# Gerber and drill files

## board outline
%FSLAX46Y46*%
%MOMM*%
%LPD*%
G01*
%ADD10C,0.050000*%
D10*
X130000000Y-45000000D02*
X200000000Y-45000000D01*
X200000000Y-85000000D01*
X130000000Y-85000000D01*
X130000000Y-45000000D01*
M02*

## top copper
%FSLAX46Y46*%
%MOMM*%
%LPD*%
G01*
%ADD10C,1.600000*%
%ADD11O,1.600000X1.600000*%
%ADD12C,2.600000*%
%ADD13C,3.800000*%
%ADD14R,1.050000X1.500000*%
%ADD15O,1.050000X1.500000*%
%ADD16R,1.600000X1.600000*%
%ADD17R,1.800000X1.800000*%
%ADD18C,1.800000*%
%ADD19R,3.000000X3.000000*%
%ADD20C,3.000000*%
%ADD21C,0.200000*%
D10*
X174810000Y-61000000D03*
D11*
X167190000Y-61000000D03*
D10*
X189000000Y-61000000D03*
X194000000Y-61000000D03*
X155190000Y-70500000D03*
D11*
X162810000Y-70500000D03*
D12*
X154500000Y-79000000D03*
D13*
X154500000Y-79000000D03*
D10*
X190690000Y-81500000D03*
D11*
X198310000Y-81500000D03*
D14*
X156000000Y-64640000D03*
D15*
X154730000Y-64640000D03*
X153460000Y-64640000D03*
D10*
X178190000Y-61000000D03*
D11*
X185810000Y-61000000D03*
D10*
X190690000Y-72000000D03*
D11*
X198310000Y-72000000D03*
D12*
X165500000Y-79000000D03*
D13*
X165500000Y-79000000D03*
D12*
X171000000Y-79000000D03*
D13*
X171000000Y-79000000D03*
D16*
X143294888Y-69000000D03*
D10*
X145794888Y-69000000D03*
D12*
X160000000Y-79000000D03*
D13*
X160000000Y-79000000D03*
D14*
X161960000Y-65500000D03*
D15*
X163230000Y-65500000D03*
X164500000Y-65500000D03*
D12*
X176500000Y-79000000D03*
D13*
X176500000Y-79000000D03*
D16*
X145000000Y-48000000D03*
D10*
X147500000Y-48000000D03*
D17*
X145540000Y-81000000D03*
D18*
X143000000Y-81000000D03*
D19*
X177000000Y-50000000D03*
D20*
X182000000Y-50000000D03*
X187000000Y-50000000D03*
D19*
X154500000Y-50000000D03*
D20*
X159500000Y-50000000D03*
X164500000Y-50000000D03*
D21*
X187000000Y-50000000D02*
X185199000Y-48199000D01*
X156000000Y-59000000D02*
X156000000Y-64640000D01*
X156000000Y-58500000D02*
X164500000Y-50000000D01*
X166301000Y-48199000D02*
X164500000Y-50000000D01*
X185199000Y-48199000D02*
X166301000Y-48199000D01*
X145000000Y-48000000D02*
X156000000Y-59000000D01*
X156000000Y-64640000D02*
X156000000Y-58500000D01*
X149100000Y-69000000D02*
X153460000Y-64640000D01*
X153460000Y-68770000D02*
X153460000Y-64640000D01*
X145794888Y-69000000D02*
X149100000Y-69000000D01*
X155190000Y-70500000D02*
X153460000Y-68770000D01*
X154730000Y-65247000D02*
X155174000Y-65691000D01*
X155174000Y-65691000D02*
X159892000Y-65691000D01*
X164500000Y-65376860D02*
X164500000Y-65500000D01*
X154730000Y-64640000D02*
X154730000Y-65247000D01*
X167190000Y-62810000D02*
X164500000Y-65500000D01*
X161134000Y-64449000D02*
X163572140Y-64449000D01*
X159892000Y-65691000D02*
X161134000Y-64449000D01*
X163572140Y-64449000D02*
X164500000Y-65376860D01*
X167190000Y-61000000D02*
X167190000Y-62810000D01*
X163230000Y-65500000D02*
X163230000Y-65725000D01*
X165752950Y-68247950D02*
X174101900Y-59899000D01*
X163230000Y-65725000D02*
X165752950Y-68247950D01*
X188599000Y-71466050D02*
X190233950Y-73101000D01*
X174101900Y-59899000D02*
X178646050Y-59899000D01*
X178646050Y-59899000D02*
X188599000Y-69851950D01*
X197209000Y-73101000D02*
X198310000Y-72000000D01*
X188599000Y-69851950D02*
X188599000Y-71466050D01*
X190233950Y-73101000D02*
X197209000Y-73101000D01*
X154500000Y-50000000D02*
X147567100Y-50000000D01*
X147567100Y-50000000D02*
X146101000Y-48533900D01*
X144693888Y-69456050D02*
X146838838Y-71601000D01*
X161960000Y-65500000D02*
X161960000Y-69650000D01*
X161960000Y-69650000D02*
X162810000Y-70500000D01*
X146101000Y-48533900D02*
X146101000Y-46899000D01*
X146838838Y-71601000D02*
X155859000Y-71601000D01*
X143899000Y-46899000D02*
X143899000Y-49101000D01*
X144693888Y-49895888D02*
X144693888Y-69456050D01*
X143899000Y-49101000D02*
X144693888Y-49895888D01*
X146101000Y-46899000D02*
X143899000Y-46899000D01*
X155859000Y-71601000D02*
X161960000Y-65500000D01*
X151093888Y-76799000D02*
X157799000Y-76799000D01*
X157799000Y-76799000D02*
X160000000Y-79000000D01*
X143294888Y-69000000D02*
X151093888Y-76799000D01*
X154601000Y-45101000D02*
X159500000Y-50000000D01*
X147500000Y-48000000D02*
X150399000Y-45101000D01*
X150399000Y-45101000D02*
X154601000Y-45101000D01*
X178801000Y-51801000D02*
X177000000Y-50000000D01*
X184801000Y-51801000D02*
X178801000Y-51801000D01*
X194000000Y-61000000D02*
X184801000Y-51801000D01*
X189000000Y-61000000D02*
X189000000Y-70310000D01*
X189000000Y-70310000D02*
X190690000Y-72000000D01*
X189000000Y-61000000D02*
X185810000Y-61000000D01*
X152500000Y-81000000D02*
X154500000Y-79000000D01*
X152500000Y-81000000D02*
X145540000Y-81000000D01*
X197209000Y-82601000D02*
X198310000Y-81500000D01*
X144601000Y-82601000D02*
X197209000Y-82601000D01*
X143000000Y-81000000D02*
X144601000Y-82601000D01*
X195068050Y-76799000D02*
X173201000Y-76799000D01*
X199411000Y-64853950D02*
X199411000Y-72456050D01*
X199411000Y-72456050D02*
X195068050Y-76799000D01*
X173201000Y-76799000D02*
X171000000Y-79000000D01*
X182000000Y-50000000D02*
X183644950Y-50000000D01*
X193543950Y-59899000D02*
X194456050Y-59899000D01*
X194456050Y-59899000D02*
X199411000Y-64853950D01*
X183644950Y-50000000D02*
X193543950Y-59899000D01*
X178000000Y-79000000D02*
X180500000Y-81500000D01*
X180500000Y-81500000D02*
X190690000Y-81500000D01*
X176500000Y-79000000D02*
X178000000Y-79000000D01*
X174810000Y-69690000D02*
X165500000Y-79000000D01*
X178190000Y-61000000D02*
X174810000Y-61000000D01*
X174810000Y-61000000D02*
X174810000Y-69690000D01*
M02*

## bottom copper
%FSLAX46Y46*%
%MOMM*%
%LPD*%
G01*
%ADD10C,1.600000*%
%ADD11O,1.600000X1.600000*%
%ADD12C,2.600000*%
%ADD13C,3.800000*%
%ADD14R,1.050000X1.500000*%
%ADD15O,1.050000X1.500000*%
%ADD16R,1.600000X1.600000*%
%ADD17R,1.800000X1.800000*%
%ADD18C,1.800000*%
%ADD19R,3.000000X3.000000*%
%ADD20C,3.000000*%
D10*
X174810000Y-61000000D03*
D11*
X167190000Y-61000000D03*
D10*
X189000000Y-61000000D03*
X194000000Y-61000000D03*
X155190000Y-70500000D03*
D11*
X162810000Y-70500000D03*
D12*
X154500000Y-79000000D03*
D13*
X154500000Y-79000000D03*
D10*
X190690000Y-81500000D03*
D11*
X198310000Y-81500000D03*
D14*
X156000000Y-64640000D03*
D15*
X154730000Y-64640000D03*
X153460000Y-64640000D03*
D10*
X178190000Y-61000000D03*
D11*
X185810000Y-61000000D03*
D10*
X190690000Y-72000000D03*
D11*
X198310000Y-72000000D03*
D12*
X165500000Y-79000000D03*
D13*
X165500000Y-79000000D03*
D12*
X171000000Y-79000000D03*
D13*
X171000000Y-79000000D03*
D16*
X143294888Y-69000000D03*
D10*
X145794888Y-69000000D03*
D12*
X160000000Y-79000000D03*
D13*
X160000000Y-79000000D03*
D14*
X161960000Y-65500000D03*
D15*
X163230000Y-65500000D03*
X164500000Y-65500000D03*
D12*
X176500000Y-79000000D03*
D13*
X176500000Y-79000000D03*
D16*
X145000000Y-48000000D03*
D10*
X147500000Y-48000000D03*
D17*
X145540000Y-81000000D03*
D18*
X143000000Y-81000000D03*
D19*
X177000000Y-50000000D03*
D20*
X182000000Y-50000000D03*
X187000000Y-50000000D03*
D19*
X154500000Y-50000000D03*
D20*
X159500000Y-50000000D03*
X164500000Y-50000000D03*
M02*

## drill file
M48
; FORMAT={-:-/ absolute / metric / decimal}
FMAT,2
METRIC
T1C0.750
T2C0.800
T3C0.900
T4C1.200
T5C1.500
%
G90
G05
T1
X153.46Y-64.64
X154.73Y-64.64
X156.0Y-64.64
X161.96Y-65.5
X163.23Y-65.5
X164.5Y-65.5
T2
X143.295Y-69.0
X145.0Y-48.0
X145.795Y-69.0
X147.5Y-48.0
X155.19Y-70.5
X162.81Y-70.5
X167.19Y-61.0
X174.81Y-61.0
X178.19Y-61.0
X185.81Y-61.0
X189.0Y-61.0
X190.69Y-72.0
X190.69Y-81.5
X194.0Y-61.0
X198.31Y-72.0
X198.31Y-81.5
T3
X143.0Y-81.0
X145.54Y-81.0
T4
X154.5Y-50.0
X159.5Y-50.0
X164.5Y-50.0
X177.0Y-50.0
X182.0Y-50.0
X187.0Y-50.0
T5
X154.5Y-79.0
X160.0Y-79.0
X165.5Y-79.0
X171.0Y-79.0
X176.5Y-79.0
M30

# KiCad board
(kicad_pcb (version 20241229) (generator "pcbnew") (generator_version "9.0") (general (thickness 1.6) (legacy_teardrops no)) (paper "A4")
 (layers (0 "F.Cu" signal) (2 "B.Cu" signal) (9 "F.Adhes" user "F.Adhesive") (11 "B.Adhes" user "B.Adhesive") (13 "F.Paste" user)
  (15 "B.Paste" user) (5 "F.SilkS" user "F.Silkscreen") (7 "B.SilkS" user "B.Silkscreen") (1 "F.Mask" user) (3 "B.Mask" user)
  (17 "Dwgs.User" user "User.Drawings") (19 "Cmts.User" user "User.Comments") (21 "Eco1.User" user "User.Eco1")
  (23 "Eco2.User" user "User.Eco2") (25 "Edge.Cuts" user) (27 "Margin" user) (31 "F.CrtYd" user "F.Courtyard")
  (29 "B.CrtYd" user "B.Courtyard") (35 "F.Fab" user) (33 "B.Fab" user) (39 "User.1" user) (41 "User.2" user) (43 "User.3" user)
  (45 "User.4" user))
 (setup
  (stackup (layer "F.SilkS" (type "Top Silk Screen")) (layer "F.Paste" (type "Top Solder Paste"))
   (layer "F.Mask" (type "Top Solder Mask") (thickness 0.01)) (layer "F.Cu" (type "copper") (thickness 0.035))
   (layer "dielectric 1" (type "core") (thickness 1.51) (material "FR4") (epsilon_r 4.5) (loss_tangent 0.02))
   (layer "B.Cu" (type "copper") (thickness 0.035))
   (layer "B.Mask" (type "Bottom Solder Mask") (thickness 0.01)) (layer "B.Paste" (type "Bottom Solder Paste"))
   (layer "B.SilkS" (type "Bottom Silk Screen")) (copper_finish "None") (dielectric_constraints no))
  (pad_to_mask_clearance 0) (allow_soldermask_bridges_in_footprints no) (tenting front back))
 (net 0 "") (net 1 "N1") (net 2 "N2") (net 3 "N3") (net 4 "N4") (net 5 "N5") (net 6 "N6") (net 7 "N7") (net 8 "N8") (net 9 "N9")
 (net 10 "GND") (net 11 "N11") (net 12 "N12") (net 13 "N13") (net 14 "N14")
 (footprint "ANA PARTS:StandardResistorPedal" (layer "F.Cu") (at 174.81 61 180)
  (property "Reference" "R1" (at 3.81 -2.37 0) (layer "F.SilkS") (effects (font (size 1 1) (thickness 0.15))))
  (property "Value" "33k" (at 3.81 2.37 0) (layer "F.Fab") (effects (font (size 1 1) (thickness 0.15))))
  (pad "1" thru_hole circle (at 0 0 180) (size 1.6 1.6) (drill 0.8) (layers "*.Cu" "*.Mask") (remove_unused_layers no) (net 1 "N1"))
  (pad "2" thru_hole oval (at 7.62 0 180) (size 1.6 1.6) (drill 0.8) (layers "*.Cu" "*.Mask") (remove_unused_layers no) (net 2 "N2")))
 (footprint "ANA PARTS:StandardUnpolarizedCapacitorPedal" (layer "F.Cu") (at 189 61)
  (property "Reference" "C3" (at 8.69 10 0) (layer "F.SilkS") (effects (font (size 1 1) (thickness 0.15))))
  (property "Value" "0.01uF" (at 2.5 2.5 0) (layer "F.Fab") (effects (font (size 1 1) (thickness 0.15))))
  (pad "1" thru_hole circle (at 0 0) (size 1.6 1.6) (drill 0.8) (layers "*.Cu" "*.Mask") (remove_unused_layers no) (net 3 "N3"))
  (pad "2" thru_hole circle (at 5 0) (size 1.6 1.6) (drill 0.8) (layers "*.Cu" "*.Mask") (remove_unused_layers no) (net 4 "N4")))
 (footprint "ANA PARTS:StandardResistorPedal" (layer "F.Cu") (at 155.19 70.5)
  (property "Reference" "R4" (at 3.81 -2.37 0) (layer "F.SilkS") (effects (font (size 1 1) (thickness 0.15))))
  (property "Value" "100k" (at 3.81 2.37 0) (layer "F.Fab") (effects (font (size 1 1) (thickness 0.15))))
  (pad "1" thru_hole circle (at 0 0) (size 1.6 1.6) (drill 0.8) (layers "*.Cu" "*.Mask") (remove_unused_layers no) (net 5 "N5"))
  (pad "2" thru_hole oval (at 7.62 0) (size 1.6 1.6) (drill 0.8) (layers "*.Cu" "*.Mask") (remove_unused_layers no) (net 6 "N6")))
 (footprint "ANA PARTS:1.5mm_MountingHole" (layer "F.Cu") (at 154.5 79)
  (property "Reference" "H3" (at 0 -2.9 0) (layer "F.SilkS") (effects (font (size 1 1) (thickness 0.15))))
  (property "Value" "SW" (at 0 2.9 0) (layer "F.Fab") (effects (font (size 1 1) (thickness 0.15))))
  (pad "1" thru_hole circle (at 0 0) (size 2.6 2.6) (drill 1.5) (layers "*.Cu" "*.Mask") (remove_unused_layers no) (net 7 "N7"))
  (pad "1" connect circle (at 0 0) (size 3.8 3.8) (layers "F.Cu" "F.Mask") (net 7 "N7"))
  (pad "1" connect circle (at 0 0) (size 3.8 3.8) (layers "B.Cu" "B.Mask") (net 7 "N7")))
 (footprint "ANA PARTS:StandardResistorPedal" (layer "F.Cu") (at 190.69 81.5)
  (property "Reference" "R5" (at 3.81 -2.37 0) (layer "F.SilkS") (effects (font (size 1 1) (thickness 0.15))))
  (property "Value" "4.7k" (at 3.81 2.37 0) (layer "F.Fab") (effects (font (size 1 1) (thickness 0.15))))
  (pad "1" thru_hole circle (at 0 0) (size 1.6 1.6) (drill 0.8) (layers "*.Cu" "*.Mask") (remove_unused_layers no) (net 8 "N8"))
  (pad "2" thru_hole oval (at 7.62 0) (size 1.6 1.6) (drill 0.8) (layers "*.Cu" "*.Mask") (remove_unused_layers no) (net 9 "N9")))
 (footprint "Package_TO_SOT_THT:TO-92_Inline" (layer "F.Cu") (at 156 64.64 180)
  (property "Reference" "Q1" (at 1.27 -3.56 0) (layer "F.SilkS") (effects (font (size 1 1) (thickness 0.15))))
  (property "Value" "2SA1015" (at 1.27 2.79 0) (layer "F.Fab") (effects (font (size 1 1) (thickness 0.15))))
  (pad "1" thru_hole rect (at 0 0 180) (size 1.05 1.5) (drill 0.75) (layers "*.Cu" "*.Mask") (remove_unused_layers no) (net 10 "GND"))
  (pad "2" thru_hole oval (at 1.27 0 180) (size 1.05 1.5) (drill 0.75) (layers "*.Cu" "*.Mask") (remove_unused_layers no) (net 2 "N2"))
  (pad "3" thru_hole oval (at 2.54 0 180) (size 1.05 1.5) (drill 0.75) (layers "*.Cu" "*.Mask") (remove_unused_layers no) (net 5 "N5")))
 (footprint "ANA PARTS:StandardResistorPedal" (layer "F.Cu") (at 178.19 61)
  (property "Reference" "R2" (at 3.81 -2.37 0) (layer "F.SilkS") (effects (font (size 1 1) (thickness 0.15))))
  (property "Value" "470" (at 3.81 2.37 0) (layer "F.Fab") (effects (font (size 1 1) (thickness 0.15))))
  (pad "1" thru_hole circle (at 0 0) (size 1.6 1.6) (drill 0.8) (layers "*.Cu" "*.Mask") (remove_unused_layers no) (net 1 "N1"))
  (pad "2" thru_hole oval (at 7.62 0) (size 1.6 1.6) (drill 0.8) (layers "*.Cu" "*.Mask") (remove_unused_layers no) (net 3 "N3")))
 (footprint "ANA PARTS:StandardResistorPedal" (layer "F.Cu") (at 190.69 72)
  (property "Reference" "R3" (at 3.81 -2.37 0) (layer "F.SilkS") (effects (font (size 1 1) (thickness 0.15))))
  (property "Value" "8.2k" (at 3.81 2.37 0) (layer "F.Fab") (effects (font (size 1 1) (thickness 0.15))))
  (pad "1" thru_hole circle (at 0 0) (size 1.6 1.6) (drill 0.8) (layers "*.Cu" "*.Mask") (remove_unused_layers no) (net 3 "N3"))
  (pad "2" thru_hole oval (at 7.62 0) (size 1.6 1.6) (drill 0.8) (layers "*.Cu" "*.Mask") (remove_unused_layers no) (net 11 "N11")))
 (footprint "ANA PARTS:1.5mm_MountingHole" (layer "F.Cu") (at 165.5 79)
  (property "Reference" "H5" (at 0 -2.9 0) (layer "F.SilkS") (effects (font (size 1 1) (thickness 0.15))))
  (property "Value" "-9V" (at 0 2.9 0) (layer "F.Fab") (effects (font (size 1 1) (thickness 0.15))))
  (pad "1" thru_hole circle (at 0 0) (size 2.6 2.6) (drill 1.5) (layers "*.Cu" "*.Mask") (remove_unused_layers no) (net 1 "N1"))
  (pad "1" connect circle (at 0 0) (size 3.8 3.8) (layers "F.Cu" "F.Mask") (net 1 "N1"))
  (pad "1" connect circle (at 0 0) (size 3.8 3.8) (layers "B.Cu" "B.Mask") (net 1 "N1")))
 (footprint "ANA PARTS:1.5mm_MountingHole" (layer "F.Cu") (at 171 79)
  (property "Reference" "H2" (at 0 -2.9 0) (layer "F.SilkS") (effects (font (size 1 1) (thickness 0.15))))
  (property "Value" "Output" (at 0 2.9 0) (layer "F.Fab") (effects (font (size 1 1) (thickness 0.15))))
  (pad "1" thru_hole circle (at 0 0) (size 2.6 2.6) (drill 1.5) (layers "*.Cu" "*.Mask") (remove_unused_layers no) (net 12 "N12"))
  (pad "1" connect circle (at 0 0) (size 3.8 3.8) (layers "F.Cu" "F.Mask") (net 12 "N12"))
  (pad "1" connect circle (at 0 0) (size 3.8 3.8) (layers "B.Cu" "B.Mask") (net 12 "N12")))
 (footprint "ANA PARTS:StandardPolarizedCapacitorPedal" (layer "F.Cu") (at 143.294888 69)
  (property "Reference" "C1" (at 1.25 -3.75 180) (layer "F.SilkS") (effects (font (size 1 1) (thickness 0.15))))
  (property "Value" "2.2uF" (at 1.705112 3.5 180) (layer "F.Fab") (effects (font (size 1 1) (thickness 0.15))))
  (pad "1" thru_hole rect (at 0 0) (size 1.6 1.6) (drill 0.8) (layers "*.Cu" "*.Mask") (remove_unused_layers no) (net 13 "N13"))
  (pad "2" thru_hole circle (at 2.5 0) (size 1.6 1.6) (drill 0.8) (layers "*.Cu" "*.Mask") (remove_unused_layers no) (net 5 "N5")))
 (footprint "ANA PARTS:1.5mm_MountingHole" (layer "F.Cu") (at 160 79)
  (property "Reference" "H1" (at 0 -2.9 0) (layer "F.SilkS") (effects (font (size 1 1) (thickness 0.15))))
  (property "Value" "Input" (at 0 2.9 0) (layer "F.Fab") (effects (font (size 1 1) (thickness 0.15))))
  (pad "1" thru_hole circle (at 0 0) (size 2.6 2.6) (drill 1.5) (layers "*.Cu" "*.Mask") (remove_unused_layers no) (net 13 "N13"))
  (pad "1" connect circle (at 0 0) (size 3.8 3.8) (layers "F.Cu" "F.Mask") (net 13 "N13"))
  (pad "1" connect circle (at 0 0) (size 3.8 3.8) (layers "B.Cu" "B.Mask") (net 13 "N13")))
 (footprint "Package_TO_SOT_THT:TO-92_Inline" (layer "F.Cu") (at 161.96 65.5)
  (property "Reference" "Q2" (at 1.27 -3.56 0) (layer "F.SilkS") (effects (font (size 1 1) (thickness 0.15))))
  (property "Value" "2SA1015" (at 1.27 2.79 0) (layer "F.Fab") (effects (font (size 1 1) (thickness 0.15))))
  (pad "1" thru_hole rect (at 0 0) (size 1.05 1.5) (drill 0.75) (layers "*.Cu" "*.Mask") (remove_unused_layers no) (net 6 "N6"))
  (pad "2" thru_hole oval (at 1.27 0) (size 1.05 1.5) (drill 0.75) (layers "*.Cu" "*.Mask") (remove_unused_layers no) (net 11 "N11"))
  (pad "3" thru_hole oval (at 2.54 0) (size 1.05 1.5) (drill 0.75) (layers "*.Cu" "*.Mask") (remove_unused_layers no) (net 2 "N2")))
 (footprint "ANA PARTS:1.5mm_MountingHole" (layer "F.Cu") (at 176.5 79)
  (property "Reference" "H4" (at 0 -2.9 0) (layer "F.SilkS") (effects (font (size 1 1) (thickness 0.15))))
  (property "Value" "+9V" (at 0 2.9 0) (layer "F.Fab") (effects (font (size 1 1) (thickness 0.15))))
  (pad "1" thru_hole circle (at 0 0) (size 2.6 2.6) (drill 1.5) (layers "*.Cu" "*.Mask") (remove_unused_layers no) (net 8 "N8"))
  (pad "1" connect circle (at 0 0) (size 3.8 3.8) (layers "F.Cu" "F.Mask") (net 8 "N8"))
  (pad "1" connect circle (at 0 0) (size 3.8 3.8) (layers "B.Cu" "B.Mask") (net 8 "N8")))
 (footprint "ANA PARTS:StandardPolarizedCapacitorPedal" (layer "F.Cu") (at 145 48)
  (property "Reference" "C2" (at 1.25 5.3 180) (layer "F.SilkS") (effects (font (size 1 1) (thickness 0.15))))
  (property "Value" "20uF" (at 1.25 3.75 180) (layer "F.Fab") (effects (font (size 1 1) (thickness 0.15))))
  (pad "1" thru_hole rect (at 0 0) (size 1.6 1.6) (drill 0.8) (layers "*.Cu" "*.Mask") (remove_unused_layers no) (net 10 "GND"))
  (pad "2" thru_hole circle (at 2.5 0) (size 1.6 1.6) (drill 0.8) (layers "*.Cu" "*.Mask") (remove_unused_layers no) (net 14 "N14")))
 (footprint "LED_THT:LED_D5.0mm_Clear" (layer "B.Cu") (at 145.54 81 180)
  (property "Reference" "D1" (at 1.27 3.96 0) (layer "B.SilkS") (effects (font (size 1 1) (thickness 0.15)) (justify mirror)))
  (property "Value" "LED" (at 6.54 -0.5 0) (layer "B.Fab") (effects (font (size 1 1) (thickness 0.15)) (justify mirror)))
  (pad "1" thru_hole rect (at 0 0 180) (size 1.8 1.8) (drill 0.9) (layers "*.Cu" "*.Mask") (remove_unused_layers no) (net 7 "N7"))
  (pad "2" thru_hole circle (at 2.54 0 180) (size 1.8 1.8) (drill 0.9) (layers "*.Cu" "*.Mask") (remove_unused_layers no) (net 9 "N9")))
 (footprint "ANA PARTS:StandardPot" (layer "B.Cu") (at 177 50 -90)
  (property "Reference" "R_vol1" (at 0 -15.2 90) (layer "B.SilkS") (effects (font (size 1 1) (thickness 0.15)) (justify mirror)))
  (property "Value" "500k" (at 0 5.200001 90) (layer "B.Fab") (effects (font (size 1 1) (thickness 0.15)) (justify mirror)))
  (pad "1" thru_hole rect (at 0 0 90) (size 3 3) (drill 1.2) (layers "*.Cu" "*.Mask") (remove_unused_layers no) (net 4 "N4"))
  (pad "2" thru_hole circle (at 0 -5 90) (size 3 3) (drill 1.2) (layers "*.Cu" "*.Mask") (remove_unused_layers no) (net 12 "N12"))
  (pad "3" thru_hole circle (at 0 -10 90) (size 3 3) (drill 1.2) (layers "*.Cu" "*.Mask") (remove_unused_layers no) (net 10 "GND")))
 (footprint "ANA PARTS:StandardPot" (layer "B.Cu") (at 154.5 50 -90)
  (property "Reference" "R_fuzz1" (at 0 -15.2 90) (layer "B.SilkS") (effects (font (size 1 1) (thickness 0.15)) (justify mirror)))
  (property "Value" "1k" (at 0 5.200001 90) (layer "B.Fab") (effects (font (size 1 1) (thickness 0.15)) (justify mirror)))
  (pad "1" thru_hole rect (at 0 0 90) (size 3 3) (drill 1.2) (layers "*.Cu" "*.Mask") (remove_unused_layers no) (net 6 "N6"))
  (pad "2" thru_hole circle (at 0 -5 90) (size 3 3) (drill 1.2) (layers "*.Cu" "*.Mask") (remove_unused_layers no) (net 14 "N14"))
  (pad "3" thru_hole circle (at 0 -10 90) (size 3 3) (drill 1.2) (layers "*.Cu" "*.Mask") (remove_unused_layers no) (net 10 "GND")))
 (gr_rect (start 130 45) (end 200 85) (stroke (width 0.05) (type solid)) (fill no) (layer "Edge.Cuts"))
 (segment (start 187 50) (end 185.199 48.199) (width 0.2) (layer "F.Cu") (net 10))
 (segment (start 156 59) (end 156 64.64) (width 0.2) (layer "F.Cu") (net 10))
 (segment (start 156 58.5) (end 164.5 50) (width 0.2) (layer "F.Cu") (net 10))
 (segment (start 166.301 48.199) (end 164.5 50) (width 0.2) (layer "F.Cu") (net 10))
 (segment (start 185.199 48.199) (end 166.301 48.199) (width 0.2) (layer "F.Cu") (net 10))
 (segment (start 145 48) (end 156 59) (width 0.2) (layer "F.Cu") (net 10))
 (segment (start 156 64.64) (end 156 58.5) (width 0.2) (layer "F.Cu") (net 10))
 (segment (start 149.1 69) (end 153.46 64.64) (width 0.2) (layer "F.Cu") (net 5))
 (segment (start 153.46 68.77) (end 153.46 64.64) (width 0.2) (layer "F.Cu") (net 5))
 (segment (start 145.794888 69) (end 149.1 69) (width 0.2) (layer "F.Cu") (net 5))
 (segment (start 155.19 70.5) (end 153.46 68.77) (width 0.2) (layer "F.Cu") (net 5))
 (segment (start 154.73 65.247) (end 155.174 65.691) (width 0.2) (layer "F.Cu") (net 2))
 (segment (start 155.174 65.691) (end 159.892 65.691) (width 0.2) (layer "F.Cu") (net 2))
 (segment (start 164.5 65.37686) (end 164.5 65.5) (width 0.2) (layer "F.Cu") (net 2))
 (segment (start 154.73 64.64) (end 154.73 65.247) (width 0.2) (layer "F.Cu") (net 2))
 (segment (start 167.19 62.81) (end 164.5 65.5) (width 0.2) (layer "F.Cu") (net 2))
 (segment (start 161.134 64.449) (end 163.57214 64.449) (width 0.2) (layer "F.Cu") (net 2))
 (segment (start 159.892 65.691) (end 161.134 64.449) (width 0.2) (layer "F.Cu") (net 2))
 (segment (start 163.57214 64.449) (end 164.5 65.37686) (width 0.2) (layer "F.Cu") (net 2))
 (segment (start 167.19 61) (end 167.19 62.81) (width 0.2) (layer "F.Cu") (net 2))
 (segment (start 163.23 65.5) (end 163.23 65.725) (width 0.2) (layer "F.Cu") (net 11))
 (segment (start 165.75295 68.24795) (end 174.1019 59.899) (width 0.2) (layer "F.Cu") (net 11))
 (segment (start 163.23 65.725) (end 165.75295 68.24795) (width 0.2) (layer "F.Cu") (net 11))
 (segment (start 188.599 71.46605) (end 190.23395 73.101) (width 0.2) (layer "F.Cu") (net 11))
 (segment (start 174.1019 59.899) (end 178.64605 59.899) (width 0.2) (layer "F.Cu") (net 11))
 (segment (start 178.64605 59.899) (end 188.599 69.85195) (width 0.2) (layer "F.Cu") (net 11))
 (segment (start 197.209 73.101) (end 198.31 72) (width 0.2) (layer "F.Cu") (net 11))
 (segment (start 188.599 69.85195) (end 188.599 71.46605) (width 0.2) (layer "F.Cu") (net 11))
 (segment (start 190.23395 73.101) (end 197.209 73.101) (width 0.2) (layer "F.Cu") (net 11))
 (segment (start 154.5 50) (end 147.5671 50) (width 0.2) (layer "F.Cu") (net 6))
 (segment (start 147.5671 50) (end 146.101 48.5339) (width 0.2) (layer "F.Cu") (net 6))
 (segment (start 144.693888 69.45605) (end 146.838838 71.601) (width 0.2) (layer "F.Cu") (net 6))
 (segment (start 161.96 65.5) (end 161.96 69.65) (width 0.2) (layer "F.Cu") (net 6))
 (segment (start 161.96 69.65) (end 162.81 70.5) (width 0.2) (layer "F.Cu") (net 6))
 (segment (start 146.101 48.5339) (end 146.101 46.899) (width 0.2) (layer "F.Cu") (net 6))
 (segment (start 146.838838 71.601) (end 155.859 71.601) (width 0.2) (layer "F.Cu") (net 6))
 (segment (start 143.899 46.899) (end 143.899 49.101) (width 0.2) (layer "F.Cu") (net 6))
 (segment (start 144.693888 49.895888) (end 144.693888 69.45605) (width 0.2) (layer "F.Cu") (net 6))
 (segment (start 143.899 49.101) (end 144.693888 49.895888) (width 0.2) (layer "F.Cu") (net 6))
 (segment (start 146.101 46.899) (end 143.899 46.899) (width 0.2) (layer "F.Cu") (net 6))
 (segment (start 155.859 71.601) (end 161.96 65.5) (width 0.2) (layer "F.Cu") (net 6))
 (segment (start 151.093888 76.799) (end 157.799 76.799) (width 0.2) (layer "F.Cu") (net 13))
 (segment (start 157.799 76.799) (end 160 79) (width 0.2) (layer "F.Cu") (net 13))
 (segment (start 143.294888 69) (end 151.093888 76.799) (width 0.2) (layer "F.Cu") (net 13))
 (segment (start 154.601 45.101) (end 159.5 50) (width 0.2) (layer "F.Cu") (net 14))
 (segment (start 147.5 48) (end 150.399 45.101) (width 0.2) (layer "F.Cu") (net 14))
 (segment (start 150.399 45.101) (end 154.601 45.101) (width 0.2) (layer "F.Cu") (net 14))
 (segment (start 178.801 51.801) (end 177 50) (width 0.2) (layer "F.Cu") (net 4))
 (segment (start 184.801 51.801) (end 178.801 51.801) (width 0.2) (layer "F.Cu") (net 4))
 (segment (start 194 61) (end 184.801 51.801) (width 0.2) (layer "F.Cu") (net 4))
 (segment (start 189 61) (end 189 70.31) (width 0.2) (layer "F.Cu") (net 3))
 (segment (start 189 70.31) (end 190.69 72) (width 0.2) (layer "F.Cu") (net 3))
 (segment (start 189 61) (end 185.81 61) (width 0.2) (layer "F.Cu") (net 3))
 (segment (start 152.5 81) (end 154.5 79) (width 0.2) (layer "F.Cu") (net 7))
 (segment (start 152.5 81) (end 145.54 81) (width 0.2) (layer "F.Cu") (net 7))
 (segment (start 197.209 82.601) (end 198.31 81.5) (width 0.2) (layer "F.Cu") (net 9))
 (segment (start 144.601 82.601) (end 197.209 82.601) (width 0.2) (layer "F.Cu") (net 9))
 (segment (start 143 81) (end 144.601 82.601) (width 0.2) (layer "F.Cu") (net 9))
 (segment (start 195.06805 76.799) (end 173.201 76.799) (width 0.2) (layer "F.Cu") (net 12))
 (segment (start 199.411 64.85395) (end 199.411 72.45605) (width 0.2) (layer "F.Cu") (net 12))
 (segment (start 199.411 72.45605) (end 195.06805 76.799) (width 0.2) (layer "F.Cu") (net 12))
 (segment (start 173.201 76.799) (end 171 79) (width 0.2) (layer "F.Cu") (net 12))
 (segment (start 182 50) (end 183.64495 50) (width 0.2) (layer "F.Cu") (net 12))
 (segment (start 193.54395 59.899) (end 194.45605 59.899) (width 0.2) (layer "F.Cu") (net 12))
 (segment (start 194.45605 59.899) (end 199.411 64.85395) (width 0.2) (layer "F.Cu") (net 12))
 (segment (start 183.64495 50) (end 193.54395 59.899) (width 0.2) (layer "F.Cu") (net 12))
 (segment (start 178 79) (end 180.5 81.5) (width 0.2) (layer "F.Cu") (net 8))
 (segment (start 180.5 81.5) (end 190.69 81.5) (width 0.2) (layer "F.Cu") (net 8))
 (segment (start 176.5 79) (end 178 79) (width 0.2) (layer "F.Cu") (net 8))
 (segment (start 174.81 69.69) (end 165.5 79) (width 0.2) (layer "F.Cu") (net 1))
 (segment (start 178.19 61) (end 174.81 61) (width 0.2) (layer "F.Cu") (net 1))
 (segment (start 174.81 61) (end 174.81 69.69) (width 0.2) (layer "F.Cu") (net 1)))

